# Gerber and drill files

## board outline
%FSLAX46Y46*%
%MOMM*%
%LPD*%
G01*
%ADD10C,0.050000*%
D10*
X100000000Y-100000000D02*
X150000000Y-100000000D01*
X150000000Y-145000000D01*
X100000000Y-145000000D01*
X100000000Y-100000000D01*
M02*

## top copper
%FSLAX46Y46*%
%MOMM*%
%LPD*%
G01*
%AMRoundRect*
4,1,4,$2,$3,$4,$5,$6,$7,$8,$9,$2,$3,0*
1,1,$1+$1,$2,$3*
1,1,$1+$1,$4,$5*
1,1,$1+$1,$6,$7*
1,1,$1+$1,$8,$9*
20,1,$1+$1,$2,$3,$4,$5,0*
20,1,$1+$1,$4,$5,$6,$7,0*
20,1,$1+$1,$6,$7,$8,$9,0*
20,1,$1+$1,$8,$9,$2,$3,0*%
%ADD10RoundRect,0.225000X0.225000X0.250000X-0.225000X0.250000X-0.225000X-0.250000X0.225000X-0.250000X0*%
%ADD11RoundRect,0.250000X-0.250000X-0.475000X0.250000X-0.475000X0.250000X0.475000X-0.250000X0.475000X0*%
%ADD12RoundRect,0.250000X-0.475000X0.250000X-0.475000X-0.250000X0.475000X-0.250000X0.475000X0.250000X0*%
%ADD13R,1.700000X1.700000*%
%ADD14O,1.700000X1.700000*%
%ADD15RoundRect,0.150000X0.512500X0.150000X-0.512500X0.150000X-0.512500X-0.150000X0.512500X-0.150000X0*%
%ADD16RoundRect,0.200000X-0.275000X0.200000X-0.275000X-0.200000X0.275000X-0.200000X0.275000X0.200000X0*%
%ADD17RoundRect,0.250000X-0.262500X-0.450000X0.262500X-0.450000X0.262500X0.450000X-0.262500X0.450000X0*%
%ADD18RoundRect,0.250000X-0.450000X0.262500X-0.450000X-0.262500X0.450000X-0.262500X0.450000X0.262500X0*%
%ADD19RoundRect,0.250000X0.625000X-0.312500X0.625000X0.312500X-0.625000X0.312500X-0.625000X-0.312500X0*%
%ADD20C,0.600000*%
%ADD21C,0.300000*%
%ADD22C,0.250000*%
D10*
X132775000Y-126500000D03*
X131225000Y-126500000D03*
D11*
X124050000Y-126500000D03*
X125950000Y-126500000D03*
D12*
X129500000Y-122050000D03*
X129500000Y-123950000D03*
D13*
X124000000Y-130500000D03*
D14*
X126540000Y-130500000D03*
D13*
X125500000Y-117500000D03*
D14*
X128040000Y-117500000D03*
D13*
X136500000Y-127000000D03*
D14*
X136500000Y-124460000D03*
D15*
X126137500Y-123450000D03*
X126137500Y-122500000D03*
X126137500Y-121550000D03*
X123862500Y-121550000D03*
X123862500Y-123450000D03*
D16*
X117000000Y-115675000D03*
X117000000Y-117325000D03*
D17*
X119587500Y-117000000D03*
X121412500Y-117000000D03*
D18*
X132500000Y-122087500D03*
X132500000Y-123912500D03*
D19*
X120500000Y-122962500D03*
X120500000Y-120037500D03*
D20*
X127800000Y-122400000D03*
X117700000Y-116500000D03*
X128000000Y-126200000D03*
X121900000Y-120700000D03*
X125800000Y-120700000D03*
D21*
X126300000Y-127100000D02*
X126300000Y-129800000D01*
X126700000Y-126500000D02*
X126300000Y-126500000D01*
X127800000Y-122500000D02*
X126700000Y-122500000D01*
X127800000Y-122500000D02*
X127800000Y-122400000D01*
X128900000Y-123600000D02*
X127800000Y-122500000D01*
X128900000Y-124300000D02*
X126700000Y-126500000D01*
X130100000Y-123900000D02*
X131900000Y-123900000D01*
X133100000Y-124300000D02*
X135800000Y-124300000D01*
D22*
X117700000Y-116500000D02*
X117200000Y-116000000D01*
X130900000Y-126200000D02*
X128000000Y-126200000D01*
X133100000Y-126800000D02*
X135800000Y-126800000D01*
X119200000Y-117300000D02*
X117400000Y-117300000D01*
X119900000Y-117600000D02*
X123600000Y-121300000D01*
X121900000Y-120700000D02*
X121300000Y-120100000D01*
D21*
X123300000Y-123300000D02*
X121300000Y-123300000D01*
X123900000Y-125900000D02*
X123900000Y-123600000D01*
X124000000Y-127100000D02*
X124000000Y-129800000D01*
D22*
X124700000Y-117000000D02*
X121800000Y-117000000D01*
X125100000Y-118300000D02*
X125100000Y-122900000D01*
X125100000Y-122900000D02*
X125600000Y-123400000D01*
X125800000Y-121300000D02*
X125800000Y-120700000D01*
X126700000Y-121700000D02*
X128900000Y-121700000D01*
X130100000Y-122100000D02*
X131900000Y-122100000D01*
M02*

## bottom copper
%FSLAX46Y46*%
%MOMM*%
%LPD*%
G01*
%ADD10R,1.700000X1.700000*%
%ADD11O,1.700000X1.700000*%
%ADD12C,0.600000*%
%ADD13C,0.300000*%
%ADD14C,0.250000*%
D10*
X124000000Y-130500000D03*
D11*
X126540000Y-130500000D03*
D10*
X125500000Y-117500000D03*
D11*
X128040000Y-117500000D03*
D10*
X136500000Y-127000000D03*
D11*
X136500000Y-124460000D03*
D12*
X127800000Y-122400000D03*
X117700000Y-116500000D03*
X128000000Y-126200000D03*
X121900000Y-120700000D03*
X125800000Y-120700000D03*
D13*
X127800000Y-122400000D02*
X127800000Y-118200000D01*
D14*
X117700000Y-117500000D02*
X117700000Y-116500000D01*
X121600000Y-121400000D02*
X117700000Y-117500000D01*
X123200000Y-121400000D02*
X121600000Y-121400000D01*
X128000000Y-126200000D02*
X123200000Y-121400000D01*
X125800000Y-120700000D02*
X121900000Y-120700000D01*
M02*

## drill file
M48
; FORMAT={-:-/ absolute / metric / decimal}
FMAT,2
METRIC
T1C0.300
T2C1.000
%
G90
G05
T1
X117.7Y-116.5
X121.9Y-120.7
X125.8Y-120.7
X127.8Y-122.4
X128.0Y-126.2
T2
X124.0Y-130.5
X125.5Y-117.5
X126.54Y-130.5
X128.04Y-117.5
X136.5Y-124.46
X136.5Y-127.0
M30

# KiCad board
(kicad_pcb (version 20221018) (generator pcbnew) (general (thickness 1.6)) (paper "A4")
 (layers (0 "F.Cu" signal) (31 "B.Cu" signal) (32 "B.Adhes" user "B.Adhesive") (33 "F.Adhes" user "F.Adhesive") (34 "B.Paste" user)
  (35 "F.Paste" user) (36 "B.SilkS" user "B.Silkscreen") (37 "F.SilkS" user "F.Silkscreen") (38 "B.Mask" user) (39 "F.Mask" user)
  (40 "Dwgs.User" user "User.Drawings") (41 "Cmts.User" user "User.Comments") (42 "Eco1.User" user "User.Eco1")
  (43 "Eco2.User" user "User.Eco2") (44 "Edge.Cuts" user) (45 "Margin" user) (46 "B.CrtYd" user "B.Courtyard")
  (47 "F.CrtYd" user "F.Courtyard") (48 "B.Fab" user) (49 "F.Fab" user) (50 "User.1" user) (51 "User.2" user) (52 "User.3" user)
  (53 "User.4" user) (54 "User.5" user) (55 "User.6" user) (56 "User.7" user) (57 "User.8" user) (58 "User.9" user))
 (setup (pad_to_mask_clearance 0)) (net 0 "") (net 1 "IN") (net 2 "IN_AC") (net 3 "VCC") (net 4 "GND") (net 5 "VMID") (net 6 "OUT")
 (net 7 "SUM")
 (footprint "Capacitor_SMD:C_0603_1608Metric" (layer "F.Cu") (at 132 126.5 180)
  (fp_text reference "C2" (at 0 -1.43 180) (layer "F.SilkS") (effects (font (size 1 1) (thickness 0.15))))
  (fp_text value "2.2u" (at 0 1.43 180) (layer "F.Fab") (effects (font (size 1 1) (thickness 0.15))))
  (pad "1" smd roundrect (at -0.775 0 180) (size 0.9 0.95) (layers "F.Cu" "F.Paste" "F.Mask") (roundrect_rratio 0.25) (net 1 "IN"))
  (pad "2" smd roundrect (at 0.775 0 180) (size 0.9 0.95) (layers "F.Cu" "F.Paste" "F.Mask") (roundrect_rratio 0.25) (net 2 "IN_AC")))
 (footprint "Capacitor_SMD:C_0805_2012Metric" (layer "F.Cu") (at 125 126.5)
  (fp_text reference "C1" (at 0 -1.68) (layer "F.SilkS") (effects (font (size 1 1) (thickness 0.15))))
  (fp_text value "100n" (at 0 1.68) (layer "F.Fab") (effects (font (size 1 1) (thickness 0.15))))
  (pad "1" smd roundrect (at -0.95 0) (size 1 1.45) (layers "F.Cu" "F.Paste" "F.Mask") (roundrect_rratio 0.25) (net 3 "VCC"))
  (pad "2" smd roundrect (at 0.95 0) (size 1 1.45) (layers "F.Cu" "F.Paste" "F.Mask") (roundrect_rratio 0.25) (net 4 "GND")))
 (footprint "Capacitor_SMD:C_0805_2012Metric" (layer "F.Cu") (at 129.5 123 -90)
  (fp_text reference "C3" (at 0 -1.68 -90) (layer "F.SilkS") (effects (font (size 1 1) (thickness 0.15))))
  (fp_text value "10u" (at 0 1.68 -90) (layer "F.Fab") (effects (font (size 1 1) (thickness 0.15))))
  (pad "1" smd roundrect (at -0.95 0 270) (size 1 1.45) (layers "F.Cu" "F.Paste" "F.Mask") (roundrect_rratio 0.25) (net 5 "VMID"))
  (pad "2" smd roundrect (at 0.95 0 270) (size 1 1.45) (layers "F.Cu" "F.Paste" "F.Mask") (roundrect_rratio 0.25) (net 4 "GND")))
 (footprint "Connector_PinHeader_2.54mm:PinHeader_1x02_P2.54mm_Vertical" (layer "F.Cu") (at 124 130.5 90)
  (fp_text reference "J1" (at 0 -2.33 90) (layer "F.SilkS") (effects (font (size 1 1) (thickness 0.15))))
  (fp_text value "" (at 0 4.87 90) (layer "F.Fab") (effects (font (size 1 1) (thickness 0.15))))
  (pad "1" thru_hole rect (at 0 0 90) (size 1.7 1.7) (drill 1) (layers "*.Cu" "*.Mask") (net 3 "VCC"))
  (pad "2" thru_hole oval (at 0 2.54 90) (size 1.7 1.7) (drill 1) (layers "*.Cu" "*.Mask") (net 4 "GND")))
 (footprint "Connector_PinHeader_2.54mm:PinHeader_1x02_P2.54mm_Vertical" (layer "F.Cu") (at 125.5 117.5 90)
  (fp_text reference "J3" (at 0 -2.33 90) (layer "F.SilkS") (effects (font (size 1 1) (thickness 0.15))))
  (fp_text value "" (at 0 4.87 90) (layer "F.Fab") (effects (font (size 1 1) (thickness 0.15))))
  (pad "1" thru_hole rect (at 0 0 90) (size 1.7 1.7) (drill 1) (layers "*.Cu" "*.Mask") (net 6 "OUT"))
  (pad "2" thru_hole oval (at 0 2.54 90) (size 1.7 1.7) (drill 1) (layers "*.Cu" "*.Mask") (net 4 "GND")))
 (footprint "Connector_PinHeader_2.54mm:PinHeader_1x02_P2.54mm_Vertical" (layer "F.Cu") (at 136.5 127 180)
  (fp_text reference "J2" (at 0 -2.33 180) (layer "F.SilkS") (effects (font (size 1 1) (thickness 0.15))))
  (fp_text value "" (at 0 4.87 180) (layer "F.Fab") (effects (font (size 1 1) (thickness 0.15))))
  (pad "1" thru_hole rect (at 0 0 180) (size 1.7 1.7) (drill 1) (layers "*.Cu" "*.Mask") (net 1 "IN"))
  (pad "2" thru_hole oval (at 0 2.54 180) (size 1.7 1.7) (drill 1) (layers "*.Cu" "*.Mask") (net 4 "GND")))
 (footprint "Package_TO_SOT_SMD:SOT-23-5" (layer "F.Cu") (at 125 122.5 180)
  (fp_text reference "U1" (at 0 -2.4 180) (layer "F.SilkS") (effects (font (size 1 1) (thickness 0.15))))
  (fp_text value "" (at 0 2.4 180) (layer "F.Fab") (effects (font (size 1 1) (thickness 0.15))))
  (pad "1" smd roundrect (at -1.1375 -0.95 180) (size 1.325 0.6) (layers "F.Cu" "F.Paste" "F.Mask") (roundrect_rratio 0.25) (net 6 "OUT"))
  (pad "2" smd roundrect (at -1.1375 0 180) (size 1.325 0.6) (layers "F.Cu" "F.Paste" "F.Mask") (roundrect_rratio 0.25) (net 4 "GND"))
  (pad "3" smd roundrect (at -1.1375 0.95 180) (size 1.325 0.6) (layers "F.Cu" "F.Paste" "F.Mask") (roundrect_rratio 0.25) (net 5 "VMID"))
  (pad "4" smd roundrect (at 1.1375 0.95 180) (size 1.325 0.6) (layers "F.Cu" "F.Paste" "F.Mask") (roundrect_rratio 0.25) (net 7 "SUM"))
  (pad "5" smd roundrect (at 1.1375 -0.95 180) (size 1.325 0.6) (layers "F.Cu" "F.Paste" "F.Mask") (roundrect_rratio 0.25) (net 3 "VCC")))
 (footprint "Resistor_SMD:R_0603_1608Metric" (layer "F.Cu") (at 117 116.5 -90)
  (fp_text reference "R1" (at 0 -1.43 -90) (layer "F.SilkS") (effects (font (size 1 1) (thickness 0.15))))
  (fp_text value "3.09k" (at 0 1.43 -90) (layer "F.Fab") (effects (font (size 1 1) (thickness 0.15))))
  (pad "1" smd roundrect (at -0.825 0 270) (size 0.8 0.95) (layers "F.Cu" "F.Paste" "F.Mask") (roundrect_rratio 0.25) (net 2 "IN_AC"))
  (pad "2" smd roundrect (at 0.825 0 270) (size 0.8 0.95) (layers "F.Cu" "F.Paste" "F.Mask") (roundrect_rratio 0.25) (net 7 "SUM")))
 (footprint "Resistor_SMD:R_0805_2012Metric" (layer "F.Cu") (at 120.5 117)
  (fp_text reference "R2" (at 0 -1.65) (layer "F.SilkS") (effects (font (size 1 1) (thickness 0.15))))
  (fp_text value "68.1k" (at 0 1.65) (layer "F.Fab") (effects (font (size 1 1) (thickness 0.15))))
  (pad "1" smd roundrect (at -0.9125 0) (size 1.025 1.4) (layers "F.Cu" "F.Paste" "F.Mask") (roundrect_rratio 0.243902) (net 7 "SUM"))
  (pad "2" smd roundrect (at 0.9125 0) (size 1.025 1.4) (layers "F.Cu" "F.Paste" "F.Mask") (roundrect_rratio 0.243902) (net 6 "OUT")))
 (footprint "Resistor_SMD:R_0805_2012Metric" (layer "F.Cu") (at 132.5 123 -90)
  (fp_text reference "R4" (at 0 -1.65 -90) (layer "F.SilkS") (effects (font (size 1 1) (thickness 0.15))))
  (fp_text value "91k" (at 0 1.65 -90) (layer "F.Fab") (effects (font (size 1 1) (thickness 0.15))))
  (pad "1" smd roundrect (at -0.9125 0 270) (size 1.025 1.4) (layers "F.Cu" "F.Paste" "F.Mask") (roundrect_rratio 0.243902) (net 5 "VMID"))
  (pad "2" smd roundrect (at 0.9125 0 270) (size 1.025 1.4) (layers "F.Cu" "F.Paste" "F.Mask") (roundrect_rratio 0.243902) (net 4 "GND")))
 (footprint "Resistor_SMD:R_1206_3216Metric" (layer "F.Cu") (at 120.5 121.5 90)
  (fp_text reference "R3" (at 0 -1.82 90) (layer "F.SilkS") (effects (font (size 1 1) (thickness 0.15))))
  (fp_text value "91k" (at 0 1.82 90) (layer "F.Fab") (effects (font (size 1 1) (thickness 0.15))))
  (pad "1" smd roundrect (at -1.4625 0 90) (size 1.125 1.75) (layers "F.Cu" "F.Paste" "F.Mask") (roundrect_rratio 0.222222) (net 3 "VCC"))
  (pad "2" smd roundrect (at 1.4625 0 90) (size 1.125 1.75) (layers "F.Cu" "F.Paste" "F.Mask") (roundrect_rratio 0.222222) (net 5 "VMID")))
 (gr_rect (start 100 100) (end 150 145) (stroke (width 0.05) (type default)) (fill none) (layer "Edge.Cuts"))
 (segment (start 126.3 127.1) (end 126.3 129.8) (width 0.3) (layer "F.Cu") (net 4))
 (segment (start 126.7 126.5) (end 126.3 126.5) (width 0.3) (layer "F.Cu") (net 4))
 (segment (start 127.8 122.5) (end 126.7 122.5) (width 0.3) (layer "F.Cu") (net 4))
 (segment (start 127.8 122.5) (end 127.8 122.4) (width 0.3) (layer "F.Cu") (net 4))
 (segment (start 128.9 123.6) (end 127.8 122.5) (width 0.3) (layer "F.Cu") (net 4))
 (segment (start 128.9 124.3) (end 126.7 126.5) (width 0.3) (layer "F.Cu") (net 4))
 (segment (start 130.1 123.9) (end 131.9 123.9) (width 0.3) (layer "F.Cu") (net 4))
 (segment (start 133.1 124.3) (end 135.8 124.3) (width 0.3) (layer "F.Cu") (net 4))
 (via (at 127.8 122.4) (size 0.6) (drill 0.3) (layers "F.Cu" "B.Cu") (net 4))
 (segment (start 117.7 116.5) (end 117.2 116) (width 0.25) (layer "F.Cu") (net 2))
 (segment (start 127.8 122.4) (end 127.8 118.2) (width 0.3) (layer "B.Cu") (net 4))
 (segment (start 130.9 126.2) (end 128 126.2) (width 0.25) (layer "F.Cu") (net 2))
 (segment (start 133.1 126.8) (end 135.8 126.8) (width 0.25) (layer "F.Cu") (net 1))
 (via (at 117.7 116.5) (size 0.6) (drill 0.3) (layers "F.Cu" "B.Cu") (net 2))
 (via (at 128 126.2) (size 0.6) (drill 0.3) (layers "F.Cu" "B.Cu") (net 2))
 (segment (start 117.7 117.5) (end 117.7 116.5) (width 0.25) (layer "B.Cu") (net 2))
 (segment (start 119.2 117.3) (end 117.4 117.3) (width 0.25) (layer "F.Cu") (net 7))
 (segment (start 119.9 117.6) (end 123.6 121.3) (width 0.25) (layer "F.Cu") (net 7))
 (segment (start 121.6 121.4) (end 117.7 117.5) (width 0.25) (layer "B.Cu") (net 2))
 (segment (start 121.9 120.7) (end 121.3 120.1) (width 0.25) (layer "F.Cu") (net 5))
 (segment (start 123.2 121.4) (end 121.6 121.4) (width 0.25) (layer "B.Cu") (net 2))
 (segment (start 123.3 123.3) (end 121.3 123.3) (width 0.3) (layer "F.Cu") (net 3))
 (segment (start 123.9 125.9) (end 123.9 123.6) (width 0.3) (layer "F.Cu") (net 3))
 (segment (start 124 127.1) (end 124 129.8) (width 0.3) (layer "F.Cu") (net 3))
 (segment (start 124.7 117) (end 121.8 117) (width 0.25) (layer "F.Cu") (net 6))
 (segment (start 125.1 118.3) (end 125.1 122.9) (width 0.25) (layer "F.Cu") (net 6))
 (segment (start 125.1 122.9) (end 125.6 123.4) (width 0.25) (layer "F.Cu") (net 6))
 (segment (start 125.8 121.3) (end 125.8 120.7) (width 0.25) (layer "F.Cu") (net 5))
 (segment (start 126.7 121.7) (end 128.9 121.7) (width 0.25) (layer "F.Cu") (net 5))
 (segment (start 128 126.2) (end 123.2 121.4) (width 0.25) (layer "B.Cu") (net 2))
 (segment (start 130.1 122.1) (end 131.9 122.1) (width 0.25) (layer "F.Cu") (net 5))
 (via (at 121.9 120.7) (size 0.6) (drill 0.3) (layers "F.Cu" "B.Cu") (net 5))
 (via (at 125.8 120.7) (size 0.6) (drill 0.3) (layers "F.Cu" "B.Cu") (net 5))
 (segment (start 125.8 120.7) (end 121.9 120.7) (width 0.25) (layer "B.Cu") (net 5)))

